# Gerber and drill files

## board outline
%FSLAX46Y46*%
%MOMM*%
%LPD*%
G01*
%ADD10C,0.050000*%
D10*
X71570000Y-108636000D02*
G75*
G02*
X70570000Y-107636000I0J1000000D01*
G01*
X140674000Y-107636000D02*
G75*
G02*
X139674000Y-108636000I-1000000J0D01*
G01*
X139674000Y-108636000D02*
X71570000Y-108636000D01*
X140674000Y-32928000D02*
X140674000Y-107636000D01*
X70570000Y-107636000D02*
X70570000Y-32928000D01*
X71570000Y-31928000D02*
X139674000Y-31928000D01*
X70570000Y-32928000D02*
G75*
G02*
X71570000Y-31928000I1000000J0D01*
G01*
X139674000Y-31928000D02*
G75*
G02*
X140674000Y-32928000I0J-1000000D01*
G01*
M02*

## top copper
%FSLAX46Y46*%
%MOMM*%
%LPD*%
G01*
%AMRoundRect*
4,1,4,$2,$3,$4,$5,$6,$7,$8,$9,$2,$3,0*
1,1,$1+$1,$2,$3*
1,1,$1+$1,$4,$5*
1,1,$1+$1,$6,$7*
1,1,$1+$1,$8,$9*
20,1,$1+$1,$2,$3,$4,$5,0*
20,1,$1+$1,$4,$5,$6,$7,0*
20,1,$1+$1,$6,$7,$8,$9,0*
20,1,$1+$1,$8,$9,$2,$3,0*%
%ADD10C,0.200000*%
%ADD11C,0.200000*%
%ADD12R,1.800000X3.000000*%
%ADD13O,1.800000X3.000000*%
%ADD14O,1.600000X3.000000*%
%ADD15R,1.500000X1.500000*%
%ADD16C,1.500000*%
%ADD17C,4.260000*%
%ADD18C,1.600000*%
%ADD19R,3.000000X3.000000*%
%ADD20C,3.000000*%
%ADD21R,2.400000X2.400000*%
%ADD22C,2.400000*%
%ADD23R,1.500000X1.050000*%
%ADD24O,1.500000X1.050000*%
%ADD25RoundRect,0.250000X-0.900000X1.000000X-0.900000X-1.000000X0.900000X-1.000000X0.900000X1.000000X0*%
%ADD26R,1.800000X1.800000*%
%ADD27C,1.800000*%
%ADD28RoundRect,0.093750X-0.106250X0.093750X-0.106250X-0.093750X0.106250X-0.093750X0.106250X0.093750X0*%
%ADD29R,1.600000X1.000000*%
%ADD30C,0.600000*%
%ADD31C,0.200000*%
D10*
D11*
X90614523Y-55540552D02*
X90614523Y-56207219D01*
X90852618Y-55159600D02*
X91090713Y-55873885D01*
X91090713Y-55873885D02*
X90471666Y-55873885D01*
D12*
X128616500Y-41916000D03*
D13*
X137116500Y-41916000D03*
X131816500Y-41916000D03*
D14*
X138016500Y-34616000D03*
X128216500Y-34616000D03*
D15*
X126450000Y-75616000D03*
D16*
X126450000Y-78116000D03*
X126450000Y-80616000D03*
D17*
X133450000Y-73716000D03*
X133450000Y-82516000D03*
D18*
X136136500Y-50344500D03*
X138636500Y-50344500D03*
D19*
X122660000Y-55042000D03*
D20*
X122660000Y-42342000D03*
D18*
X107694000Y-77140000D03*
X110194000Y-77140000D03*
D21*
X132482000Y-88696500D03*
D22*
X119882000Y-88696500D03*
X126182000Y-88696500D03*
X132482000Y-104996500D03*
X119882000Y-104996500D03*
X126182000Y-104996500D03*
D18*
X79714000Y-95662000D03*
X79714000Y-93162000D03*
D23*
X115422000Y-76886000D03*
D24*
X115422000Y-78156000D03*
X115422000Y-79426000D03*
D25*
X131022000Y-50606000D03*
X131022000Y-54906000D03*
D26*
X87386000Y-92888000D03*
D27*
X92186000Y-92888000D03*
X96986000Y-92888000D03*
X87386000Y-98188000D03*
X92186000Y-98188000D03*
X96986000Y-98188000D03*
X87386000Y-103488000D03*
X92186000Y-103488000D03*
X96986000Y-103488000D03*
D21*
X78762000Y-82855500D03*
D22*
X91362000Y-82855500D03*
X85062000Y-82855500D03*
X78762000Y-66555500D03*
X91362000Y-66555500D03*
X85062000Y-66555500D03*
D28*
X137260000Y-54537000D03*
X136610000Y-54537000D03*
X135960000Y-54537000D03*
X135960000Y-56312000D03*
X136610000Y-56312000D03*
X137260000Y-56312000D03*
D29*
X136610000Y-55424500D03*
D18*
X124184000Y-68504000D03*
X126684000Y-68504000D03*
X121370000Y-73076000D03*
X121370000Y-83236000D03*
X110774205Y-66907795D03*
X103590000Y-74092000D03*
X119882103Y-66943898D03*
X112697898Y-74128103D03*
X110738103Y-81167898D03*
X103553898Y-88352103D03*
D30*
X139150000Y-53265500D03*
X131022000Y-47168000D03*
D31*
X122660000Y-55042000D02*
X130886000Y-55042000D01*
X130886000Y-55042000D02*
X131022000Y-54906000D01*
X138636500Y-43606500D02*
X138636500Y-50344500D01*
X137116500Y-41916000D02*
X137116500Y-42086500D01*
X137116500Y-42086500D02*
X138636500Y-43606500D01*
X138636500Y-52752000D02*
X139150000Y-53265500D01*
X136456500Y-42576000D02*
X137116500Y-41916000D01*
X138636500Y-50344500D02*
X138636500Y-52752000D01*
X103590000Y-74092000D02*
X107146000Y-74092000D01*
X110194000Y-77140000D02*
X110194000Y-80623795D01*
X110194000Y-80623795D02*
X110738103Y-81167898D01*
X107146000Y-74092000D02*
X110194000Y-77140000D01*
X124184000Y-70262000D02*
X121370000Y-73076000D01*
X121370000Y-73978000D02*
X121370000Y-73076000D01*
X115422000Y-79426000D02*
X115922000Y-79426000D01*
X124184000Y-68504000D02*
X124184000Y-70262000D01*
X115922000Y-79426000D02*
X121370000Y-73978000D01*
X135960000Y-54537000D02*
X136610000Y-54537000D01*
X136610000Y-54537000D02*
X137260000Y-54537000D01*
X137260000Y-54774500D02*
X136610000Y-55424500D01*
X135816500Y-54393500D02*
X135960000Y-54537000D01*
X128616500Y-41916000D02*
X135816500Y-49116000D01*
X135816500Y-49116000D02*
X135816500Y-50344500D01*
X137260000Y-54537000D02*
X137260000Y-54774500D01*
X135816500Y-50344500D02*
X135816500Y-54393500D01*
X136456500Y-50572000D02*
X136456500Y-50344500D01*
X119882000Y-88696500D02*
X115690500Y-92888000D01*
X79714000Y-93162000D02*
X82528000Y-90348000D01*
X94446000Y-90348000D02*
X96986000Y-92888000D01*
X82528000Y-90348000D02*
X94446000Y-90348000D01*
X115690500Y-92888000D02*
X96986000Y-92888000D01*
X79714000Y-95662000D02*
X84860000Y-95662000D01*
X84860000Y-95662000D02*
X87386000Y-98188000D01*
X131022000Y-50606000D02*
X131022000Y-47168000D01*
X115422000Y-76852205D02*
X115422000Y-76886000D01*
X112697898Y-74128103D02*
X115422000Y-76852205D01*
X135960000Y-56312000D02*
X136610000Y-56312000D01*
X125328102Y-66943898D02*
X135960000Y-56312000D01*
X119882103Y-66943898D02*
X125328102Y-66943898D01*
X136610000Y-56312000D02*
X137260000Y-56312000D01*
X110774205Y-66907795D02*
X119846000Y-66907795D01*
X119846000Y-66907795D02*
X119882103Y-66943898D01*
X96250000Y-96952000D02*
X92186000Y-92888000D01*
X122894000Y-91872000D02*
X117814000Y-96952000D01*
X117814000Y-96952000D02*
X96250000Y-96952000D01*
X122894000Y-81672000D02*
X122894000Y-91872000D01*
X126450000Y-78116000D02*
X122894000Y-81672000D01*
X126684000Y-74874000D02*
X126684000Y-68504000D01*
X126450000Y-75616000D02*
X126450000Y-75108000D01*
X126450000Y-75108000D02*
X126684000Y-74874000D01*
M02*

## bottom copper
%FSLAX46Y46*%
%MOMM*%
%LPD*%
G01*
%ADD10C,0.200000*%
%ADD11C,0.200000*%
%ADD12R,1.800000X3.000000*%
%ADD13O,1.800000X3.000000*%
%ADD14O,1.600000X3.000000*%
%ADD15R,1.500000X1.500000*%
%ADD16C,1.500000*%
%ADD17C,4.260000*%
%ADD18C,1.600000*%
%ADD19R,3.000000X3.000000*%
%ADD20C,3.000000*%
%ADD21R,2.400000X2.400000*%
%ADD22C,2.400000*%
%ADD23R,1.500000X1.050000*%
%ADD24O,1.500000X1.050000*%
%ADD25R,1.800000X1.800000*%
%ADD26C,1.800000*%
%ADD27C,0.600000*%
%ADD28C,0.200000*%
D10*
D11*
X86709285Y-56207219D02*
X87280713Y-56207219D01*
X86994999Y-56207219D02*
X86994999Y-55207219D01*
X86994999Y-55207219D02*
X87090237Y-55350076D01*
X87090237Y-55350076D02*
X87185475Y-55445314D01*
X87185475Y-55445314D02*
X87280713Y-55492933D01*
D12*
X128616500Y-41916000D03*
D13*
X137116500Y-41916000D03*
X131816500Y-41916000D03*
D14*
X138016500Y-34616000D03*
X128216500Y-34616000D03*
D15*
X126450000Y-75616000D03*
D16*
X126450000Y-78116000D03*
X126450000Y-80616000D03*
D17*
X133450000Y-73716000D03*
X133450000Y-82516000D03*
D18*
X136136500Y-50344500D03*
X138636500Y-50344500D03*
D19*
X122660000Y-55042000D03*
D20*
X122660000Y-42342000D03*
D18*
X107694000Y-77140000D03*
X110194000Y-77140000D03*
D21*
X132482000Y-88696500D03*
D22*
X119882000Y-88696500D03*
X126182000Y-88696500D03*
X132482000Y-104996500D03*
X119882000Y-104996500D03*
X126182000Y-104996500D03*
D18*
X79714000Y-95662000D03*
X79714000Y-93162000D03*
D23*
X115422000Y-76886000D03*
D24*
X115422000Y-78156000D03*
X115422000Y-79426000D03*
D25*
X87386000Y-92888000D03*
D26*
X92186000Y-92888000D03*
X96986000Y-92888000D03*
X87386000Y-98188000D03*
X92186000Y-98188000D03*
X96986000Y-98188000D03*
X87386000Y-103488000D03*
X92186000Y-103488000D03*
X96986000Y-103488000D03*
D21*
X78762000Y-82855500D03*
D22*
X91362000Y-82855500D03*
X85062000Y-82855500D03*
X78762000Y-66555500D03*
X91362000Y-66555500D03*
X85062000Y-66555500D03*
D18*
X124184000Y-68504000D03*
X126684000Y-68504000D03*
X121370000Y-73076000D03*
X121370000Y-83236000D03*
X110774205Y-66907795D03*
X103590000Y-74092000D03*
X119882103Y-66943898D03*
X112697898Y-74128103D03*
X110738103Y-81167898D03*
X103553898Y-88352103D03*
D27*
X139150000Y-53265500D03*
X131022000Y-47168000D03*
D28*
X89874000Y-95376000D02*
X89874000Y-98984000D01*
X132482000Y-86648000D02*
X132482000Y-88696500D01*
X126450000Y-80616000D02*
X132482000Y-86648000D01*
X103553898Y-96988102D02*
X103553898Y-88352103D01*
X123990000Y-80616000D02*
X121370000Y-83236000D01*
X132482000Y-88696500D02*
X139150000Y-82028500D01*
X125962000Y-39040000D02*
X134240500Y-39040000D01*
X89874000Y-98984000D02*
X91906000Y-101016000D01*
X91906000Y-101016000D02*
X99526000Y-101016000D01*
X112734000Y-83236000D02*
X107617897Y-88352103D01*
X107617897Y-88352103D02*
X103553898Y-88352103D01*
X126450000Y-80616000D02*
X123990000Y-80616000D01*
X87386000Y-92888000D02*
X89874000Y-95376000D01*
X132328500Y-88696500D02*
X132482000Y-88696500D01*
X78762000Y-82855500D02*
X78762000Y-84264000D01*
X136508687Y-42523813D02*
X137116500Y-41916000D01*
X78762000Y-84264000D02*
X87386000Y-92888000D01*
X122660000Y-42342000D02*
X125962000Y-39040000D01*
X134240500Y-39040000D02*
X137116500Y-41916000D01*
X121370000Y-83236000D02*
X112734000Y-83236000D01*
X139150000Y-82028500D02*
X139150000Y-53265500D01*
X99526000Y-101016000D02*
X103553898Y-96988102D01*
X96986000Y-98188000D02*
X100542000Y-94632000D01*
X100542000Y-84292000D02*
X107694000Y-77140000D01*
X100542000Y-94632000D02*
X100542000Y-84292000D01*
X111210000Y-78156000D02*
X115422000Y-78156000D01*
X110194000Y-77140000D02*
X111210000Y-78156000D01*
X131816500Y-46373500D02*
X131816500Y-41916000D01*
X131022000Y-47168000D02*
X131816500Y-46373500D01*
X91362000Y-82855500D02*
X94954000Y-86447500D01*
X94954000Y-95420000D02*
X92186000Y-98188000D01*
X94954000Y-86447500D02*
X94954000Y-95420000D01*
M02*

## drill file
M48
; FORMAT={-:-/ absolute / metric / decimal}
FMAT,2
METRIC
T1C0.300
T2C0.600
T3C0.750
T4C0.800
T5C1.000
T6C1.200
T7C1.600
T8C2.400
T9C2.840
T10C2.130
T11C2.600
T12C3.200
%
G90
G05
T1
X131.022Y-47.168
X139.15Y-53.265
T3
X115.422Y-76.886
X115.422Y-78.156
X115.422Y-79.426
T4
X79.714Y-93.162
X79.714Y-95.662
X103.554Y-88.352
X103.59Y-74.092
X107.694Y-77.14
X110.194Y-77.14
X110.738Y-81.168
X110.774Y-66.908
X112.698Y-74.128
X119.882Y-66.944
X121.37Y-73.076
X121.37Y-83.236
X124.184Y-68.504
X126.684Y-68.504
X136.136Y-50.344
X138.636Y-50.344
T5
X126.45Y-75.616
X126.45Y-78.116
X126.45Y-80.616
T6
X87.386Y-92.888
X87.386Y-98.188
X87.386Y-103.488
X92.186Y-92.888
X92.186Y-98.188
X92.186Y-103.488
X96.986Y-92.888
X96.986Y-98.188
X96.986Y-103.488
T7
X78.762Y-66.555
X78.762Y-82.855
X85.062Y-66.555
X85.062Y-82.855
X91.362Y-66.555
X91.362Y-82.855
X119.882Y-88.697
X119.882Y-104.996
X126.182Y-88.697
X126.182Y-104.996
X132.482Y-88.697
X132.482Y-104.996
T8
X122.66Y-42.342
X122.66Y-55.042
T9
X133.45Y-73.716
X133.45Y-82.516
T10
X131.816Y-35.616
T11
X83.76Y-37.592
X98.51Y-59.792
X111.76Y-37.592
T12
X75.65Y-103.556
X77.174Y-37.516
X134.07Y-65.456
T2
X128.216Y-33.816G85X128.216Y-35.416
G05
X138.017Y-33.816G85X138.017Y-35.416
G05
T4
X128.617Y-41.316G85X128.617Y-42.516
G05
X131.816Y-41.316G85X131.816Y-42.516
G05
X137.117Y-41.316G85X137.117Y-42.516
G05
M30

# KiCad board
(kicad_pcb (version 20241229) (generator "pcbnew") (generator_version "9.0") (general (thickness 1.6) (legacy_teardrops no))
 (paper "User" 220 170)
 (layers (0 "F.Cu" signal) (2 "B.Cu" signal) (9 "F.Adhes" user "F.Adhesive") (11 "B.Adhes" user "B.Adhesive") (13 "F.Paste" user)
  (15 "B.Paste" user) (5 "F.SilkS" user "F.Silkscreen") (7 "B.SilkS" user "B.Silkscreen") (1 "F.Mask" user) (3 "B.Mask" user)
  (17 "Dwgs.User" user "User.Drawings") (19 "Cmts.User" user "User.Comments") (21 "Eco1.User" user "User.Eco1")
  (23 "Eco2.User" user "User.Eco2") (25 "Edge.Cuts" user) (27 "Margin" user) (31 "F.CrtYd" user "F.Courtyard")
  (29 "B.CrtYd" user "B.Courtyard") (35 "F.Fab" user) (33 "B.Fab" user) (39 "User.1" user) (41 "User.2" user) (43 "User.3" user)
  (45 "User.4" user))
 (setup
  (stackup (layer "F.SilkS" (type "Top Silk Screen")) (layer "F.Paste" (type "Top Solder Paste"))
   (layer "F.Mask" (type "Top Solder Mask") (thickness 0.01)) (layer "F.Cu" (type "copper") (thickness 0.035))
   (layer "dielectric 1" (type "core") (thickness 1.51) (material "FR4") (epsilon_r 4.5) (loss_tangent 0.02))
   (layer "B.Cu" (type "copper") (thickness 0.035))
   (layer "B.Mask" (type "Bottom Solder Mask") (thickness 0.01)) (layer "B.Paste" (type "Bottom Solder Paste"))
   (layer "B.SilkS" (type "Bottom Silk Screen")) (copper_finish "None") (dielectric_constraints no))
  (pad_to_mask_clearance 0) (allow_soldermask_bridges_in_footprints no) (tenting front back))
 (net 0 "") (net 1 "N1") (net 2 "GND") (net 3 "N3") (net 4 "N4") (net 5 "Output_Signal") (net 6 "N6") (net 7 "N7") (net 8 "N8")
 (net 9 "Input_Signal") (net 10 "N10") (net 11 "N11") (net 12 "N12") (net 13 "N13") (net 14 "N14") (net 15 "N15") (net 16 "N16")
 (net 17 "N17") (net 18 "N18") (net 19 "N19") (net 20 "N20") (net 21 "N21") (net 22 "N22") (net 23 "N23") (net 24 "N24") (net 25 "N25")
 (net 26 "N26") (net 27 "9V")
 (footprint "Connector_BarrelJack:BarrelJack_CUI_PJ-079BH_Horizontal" (layer "F.Cu") (at 128.6165 41.916 180)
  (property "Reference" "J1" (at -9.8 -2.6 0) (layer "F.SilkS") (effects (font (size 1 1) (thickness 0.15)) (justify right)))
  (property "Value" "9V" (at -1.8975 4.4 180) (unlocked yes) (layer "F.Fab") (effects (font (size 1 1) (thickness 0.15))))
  (pad "" np_thru_hole circle (at -3.2 6.3) (size 2.13 2.13) (drill 2.13) (layers "*.Cu" "*.Mask"))
  (pad "1" thru_hole rect (at 0 0) (size 1.8 3) (drill oval 0.8 2) (layers "*.Cu" "*.Mask") (remove_unused_layers no) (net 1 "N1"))
  (pad "2" thru_hole oval (at -8.5 0) (size 1.8 3) (drill oval 0.8 2) (layers "*.Cu" "*.Mask") (remove_unused_layers no) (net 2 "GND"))
  (pad "3" thru_hole oval (at -3.2 0) (size 1.8 3) (drill oval 0.8 2) (layers "*.Cu" "*.Mask") (remove_unused_layers no) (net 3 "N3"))
  (pad "SH" thru_hole oval (at -9.4 7.3) (size 1.6 3) (drill oval 0.6 2.2) (layers "*.Cu" "*.Mask") (remove_unused_layers no))
  (pad "SH" thru_hole oval (at 0.4 7.3) (size 1.6 3) (drill oval 0.6 2.2) (layers "*.Cu" "*.Mask") (remove_unused_layers no)))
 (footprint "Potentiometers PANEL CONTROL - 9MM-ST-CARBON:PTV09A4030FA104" (layer "F.Cu") (at 126.45 75.616 -90)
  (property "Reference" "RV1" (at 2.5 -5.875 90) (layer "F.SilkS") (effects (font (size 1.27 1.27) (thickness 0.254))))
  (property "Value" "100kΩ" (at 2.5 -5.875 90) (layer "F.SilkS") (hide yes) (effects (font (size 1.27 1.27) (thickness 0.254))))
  (pad "1" thru_hole rect (at 0 0 270) (size 1.5 1.5) (drill 1) (layers "*.Cu" "*.Mask") (remove_unused_layers no) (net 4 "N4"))
  (pad "2" thru_hole circle (at 2.5 0 270) (size 1.5 1.5) (drill 1) (layers "*.Cu" "*.Mask") (remove_unused_layers no)
   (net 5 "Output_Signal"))
  (pad "3" thru_hole circle (at 5 0 270) (size 1.5 1.5) (drill 1) (layers "*.Cu" "*.Mask") (remove_unused_layers no) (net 2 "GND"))
  (pad "4" thru_hole circle (at -1.9 -7 270) (size 4.26 4.26) (drill 2.84) (layers "*.Cu" "*.Mask") (remove_unused_layers no) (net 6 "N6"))
  (pad "5" thru_hole circle (at 6.9 -7 270) (size 4.26 4.26) (drill 2.84) (layers "*.Cu" "*.Mask") (remove_unused_layers no) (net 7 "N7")))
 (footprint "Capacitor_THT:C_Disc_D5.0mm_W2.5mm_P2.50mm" (layer "F.Cu") (at 136.1365 50.3445)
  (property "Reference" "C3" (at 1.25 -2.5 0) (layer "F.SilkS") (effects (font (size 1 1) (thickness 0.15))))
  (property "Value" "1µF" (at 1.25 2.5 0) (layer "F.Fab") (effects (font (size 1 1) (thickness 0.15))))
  (pad "1" thru_hole circle (at 0 0) (size 1.6 1.6) (drill 0.8) (layers "*.Cu" "*.Mask") (remove_unused_layers no) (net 1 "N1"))
  (pad "2" thru_hole circle (at 2.5 0) (size 1.6 1.6) (drill 0.8) (layers "*.Cu" "*.Mask") (remove_unused_layers no) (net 2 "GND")))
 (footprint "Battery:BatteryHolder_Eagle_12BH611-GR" (layer "F.Cu") (at 122.66 55.042)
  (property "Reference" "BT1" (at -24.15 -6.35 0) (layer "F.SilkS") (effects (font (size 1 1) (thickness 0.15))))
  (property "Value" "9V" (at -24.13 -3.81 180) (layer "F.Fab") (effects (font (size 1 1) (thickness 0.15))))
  (pad "" np_thru_hole circle (at -38.9 -17.45) (size 2.6 2.6) (drill 2.6) (layers "*.Cu" "*.Mask"))
  (pad "" np_thru_hole circle (at -24.15 4.75) (size 2.6 2.6) (drill 2.6) (layers "*.Cu" "*.Mask"))
  (pad "" np_thru_hole circle (at -10.9 -17.45) (size 2.6 2.6) (drill 2.6) (layers "*.Cu" "*.Mask"))
  (pad "1" thru_hole rect (at 0 0) (size 3 3) (drill 2.4) (layers "*.Cu" "*.Mask") (remove_unused_layers no) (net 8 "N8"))
  (pad "2" thru_hole circle (at 0 -12.7) (size 3 3) (drill 2.4) (layers "*.Cu" "*.Mask") (remove_unused_layers no) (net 2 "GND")))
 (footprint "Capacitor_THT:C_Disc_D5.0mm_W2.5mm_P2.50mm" (layer "F.Cu") (at 107.694 77.14)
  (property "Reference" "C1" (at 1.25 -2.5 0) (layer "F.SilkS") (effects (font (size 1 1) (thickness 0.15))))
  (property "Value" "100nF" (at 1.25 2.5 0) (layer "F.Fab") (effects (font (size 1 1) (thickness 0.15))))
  (pad "1" thru_hole circle (at 0 0) (size 1.6 1.6) (drill 0.8) (layers "*.Cu" "*.Mask") (remove_unused_layers no) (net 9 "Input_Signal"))
  (pad "2" thru_hole circle (at 2.5 0) (size 1.6 1.6) (drill 0.8) (layers "*.Cu" "*.Mask") (remove_unused_layers no) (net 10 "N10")))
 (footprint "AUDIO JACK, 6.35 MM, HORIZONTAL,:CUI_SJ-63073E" (layer "F.Cu") (at 132.482 96.8465 180)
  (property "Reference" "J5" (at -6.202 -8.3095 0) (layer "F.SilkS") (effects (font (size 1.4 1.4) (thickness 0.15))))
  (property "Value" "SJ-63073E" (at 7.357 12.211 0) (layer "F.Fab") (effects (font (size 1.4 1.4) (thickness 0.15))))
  (pad "1" thru_hole rect (at 0 8.15 180) (size 2.4 2.4) (drill 1.6) (layers "*.Cu" "*.Mask") (remove_unused_layers no) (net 2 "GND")
   (solder_mask_margin 0.102))
  (pad "2" thru_hole circle (at 12.6 8.15 180) (size 2.4 2.4) (drill 1.6) (layers "*.Cu" "*.Mask") (remove_unused_layers no) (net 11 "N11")
   (solder_mask_margin 0.102))
  (pad "3" thru_hole circle (at 6.3 8.15 180) (size 2.4 2.4) (drill 1.6) (layers "*.Cu" "*.Mask") (remove_unused_layers no) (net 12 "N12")
   (solder_mask_margin 0.102))
  (pad "4" thru_hole circle (at 0 -8.15 180) (size 2.4 2.4) (drill 1.6) (layers "*.Cu" "*.Mask") (remove_unused_layers no) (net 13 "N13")
   (solder_mask_margin 0.102))
  (pad "5" thru_hole circle (at 12.6 -8.15 180) (size 2.4 2.4) (drill 1.6) (layers "*.Cu" "*.Mask") (remove_unused_layers no) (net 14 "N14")
   (solder_mask_margin 0.102))
  (pad "6" thru_hole circle (at 6.3 -8.15 180) (size 2.4 2.4) (drill 1.6) (layers "*.Cu" "*.Mask") (remove_unused_layers no) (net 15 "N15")
   (solder_mask_margin 0.102)))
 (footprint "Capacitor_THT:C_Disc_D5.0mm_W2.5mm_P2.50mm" (layer "F.Cu") (at 79.714 95.662 90)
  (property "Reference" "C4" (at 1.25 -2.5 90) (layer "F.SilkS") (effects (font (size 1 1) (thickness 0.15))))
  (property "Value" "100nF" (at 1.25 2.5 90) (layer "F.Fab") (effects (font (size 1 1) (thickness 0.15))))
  (pad "1" thru_hole circle (at 0 0 90) (size 1.6 1.6) (drill 0.8) (layers "*.Cu" "*.Mask") (remove_unused_layers no) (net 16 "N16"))
  (pad "2" thru_hole circle (at 2.5 0 90) (size 1.6 1.6) (drill 0.8) (layers "*.Cu" "*.Mask") (remove_unused_layers no) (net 11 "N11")))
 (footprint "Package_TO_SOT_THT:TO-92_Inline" (layer "F.Cu") (at 115.422 76.886 -90)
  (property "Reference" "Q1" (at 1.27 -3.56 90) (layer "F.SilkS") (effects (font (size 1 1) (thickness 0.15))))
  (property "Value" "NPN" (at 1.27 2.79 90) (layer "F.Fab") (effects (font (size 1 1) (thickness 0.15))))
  (pad "1" thru_hole rect (at 0 0 270) (size 1.05 1.5) (drill 0.75) (layers "*.Cu" "*.Mask") (remove_unused_layers no) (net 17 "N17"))
  (pad "2" thru_hole oval (at 1.27 0 270) (size 1.05 1.5) (drill 0.75) (layers "*.Cu" "*.Mask") (remove_unused_layers no) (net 10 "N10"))
  (pad "3" thru_hole oval (at 2.54 0 270) (size 1.05 1.5) (drill 0.75) (layers "*.Cu" "*.Mask") (remove_unused_layers no) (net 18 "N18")))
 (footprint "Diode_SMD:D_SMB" (layer "F.Cu") (at 131.022 52.756 -90)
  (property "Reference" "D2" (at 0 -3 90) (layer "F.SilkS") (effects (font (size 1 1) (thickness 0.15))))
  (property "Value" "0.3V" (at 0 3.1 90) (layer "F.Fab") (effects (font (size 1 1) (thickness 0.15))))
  (pad "1" smd roundrect (at -2.15 0 270) (size 2.5 2.3) (layers "F.Cu" "F.Mask" "F.Paste") (roundrect_rratio 0.1086956522) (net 3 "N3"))
  (pad "2" smd roundrect (at 2.15 0 270) (size 2.5 2.3) (layers "F.Cu" "F.Mask" "F.Paste") (roundrect_rratio 0.1086956522) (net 8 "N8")))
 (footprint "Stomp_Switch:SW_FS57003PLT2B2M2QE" (layer "F.Cu") (at 92.186 98.188 -90)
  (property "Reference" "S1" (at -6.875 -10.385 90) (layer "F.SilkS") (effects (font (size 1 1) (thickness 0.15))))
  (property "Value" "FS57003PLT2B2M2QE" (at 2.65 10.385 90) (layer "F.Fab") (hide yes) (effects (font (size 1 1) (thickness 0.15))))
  (pad "1" thru_hole rect (at -5.3 4.8 270) (size 1.8 1.8) (drill 1.2) (layers "*.Cu" "*.Mask") (remove_unused_layers no) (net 2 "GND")
   (solder_mask_margin 0.102))
  (pad "2" thru_hole circle (at -5.3 0 270) (size 1.8 1.8) (drill 1.2) (layers "*.Cu" "*.Mask") (remove_unused_layers no)
   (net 5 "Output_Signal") (solder_mask_margin 0.102))
  (pad "3" thru_hole circle (at -5.3 -4.8 270) (size 1.8 1.8) (drill 1.2) (layers "*.Cu" "*.Mask") (remove_unused_layers no) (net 11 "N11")
   (solder_mask_margin 0.102))
  (pad "4" thru_hole circle (at 0 4.8 270) (size 1.8 1.8) (drill 1.2) (layers "*.Cu" "*.Mask") (remove_unused_layers no) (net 16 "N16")
   (solder_mask_margin 0.102))
  (pad "5" thru_hole circle (at 0 0 270) (size 1.8 1.8) (drill 1.2) (layers "*.Cu" "*.Mask") (remove_unused_layers no) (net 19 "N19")
   (solder_mask_margin 0.102))
  (pad "6" thru_hole circle (at 0 -4.8 270) (size 1.8 1.8) (drill 1.2) (layers "*.Cu" "*.Mask") (remove_unused_layers no)
   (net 9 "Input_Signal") (solder_mask_margin 0.102))
  (pad "7" thru_hole circle (at 5.3 4.8 270) (size 1.8 1.8) (drill 1.2) (layers "*.Cu" "*.Mask") (remove_unused_layers no) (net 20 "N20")
   (solder_mask_margin 0.102))
  (pad "8" thru_hole circle (at 5.3 0 270) (size 1.8 1.8) (drill 1.2) (layers "*.Cu" "*.Mask") (remove_unused_layers no) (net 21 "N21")
   (solder_mask_margin 0.102))
  (pad "9" thru_hole circle (at 5.3 -4.8 270) (size 1.8 1.8) (drill 1.2) (layers "*.Cu" "*.Mask") (remove_unused_layers no) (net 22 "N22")
   (solder_mask_margin 0.102)))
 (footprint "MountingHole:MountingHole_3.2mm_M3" (layer "F.Cu") (at 75.65 103.556)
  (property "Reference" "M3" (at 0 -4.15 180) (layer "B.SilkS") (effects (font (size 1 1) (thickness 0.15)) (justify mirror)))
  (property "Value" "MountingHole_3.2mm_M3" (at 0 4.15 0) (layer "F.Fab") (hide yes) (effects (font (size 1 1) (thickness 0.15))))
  (pad "" np_thru_hole circle (at 0 0) (size 3.2 3.2) (drill 3.2) (layers "*.Cu" "*.Mask")))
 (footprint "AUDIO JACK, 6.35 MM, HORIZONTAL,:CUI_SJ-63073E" (layer "F.Cu") (at 78.762 74.7055)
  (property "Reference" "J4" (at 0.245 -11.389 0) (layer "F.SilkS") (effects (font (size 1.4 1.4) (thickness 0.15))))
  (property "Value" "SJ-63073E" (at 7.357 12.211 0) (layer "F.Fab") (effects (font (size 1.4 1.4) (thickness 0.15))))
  (pad "1" thru_hole rect (at 0 8.15) (size 2.4 2.4) (drill 1.6) (layers "*.Cu" "*.Mask") (remove_unused_layers no) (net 2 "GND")
   (solder_mask_margin 0.102))
  (pad "2" thru_hole circle (at 12.6 8.15) (size 2.4 2.4) (drill 1.6) (layers "*.Cu" "*.Mask") (remove_unused_layers no) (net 19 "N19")
   (solder_mask_margin 0.102))
  (pad "3" thru_hole circle (at 6.3 8.15) (size 2.4 2.4) (drill 1.6) (layers "*.Cu" "*.Mask") (remove_unused_layers no) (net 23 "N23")
   (solder_mask_margin 0.102))
  (pad "4" thru_hole circle (at 0 -8.15) (size 2.4 2.4) (drill 1.6) (layers "*.Cu" "*.Mask") (remove_unused_layers no) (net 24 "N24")
   (solder_mask_margin 0.102))
  (pad "5" thru_hole circle (at 12.6 -8.15) (size 2.4 2.4) (drill 1.6) (layers "*.Cu" "*.Mask") (remove_unused_layers no) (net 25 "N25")
   (solder_mask_margin 0.102))
  (pad "6" thru_hole circle (at 6.3 -8.15) (size 2.4 2.4) (drill 1.6) (layers "*.Cu" "*.Mask") (remove_unused_layers no) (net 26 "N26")
   (solder_mask_margin 0.102)))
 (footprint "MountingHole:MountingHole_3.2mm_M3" (layer "F.Cu") (at 134.07 65.456)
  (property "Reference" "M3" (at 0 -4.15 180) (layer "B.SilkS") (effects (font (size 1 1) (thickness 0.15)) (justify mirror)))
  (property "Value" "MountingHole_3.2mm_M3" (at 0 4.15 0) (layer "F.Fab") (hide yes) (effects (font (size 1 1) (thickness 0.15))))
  (pad "" np_thru_hole circle (at 0 0) (size 3.2 3.2) (drill 3.2) (layers "*.Cu" "*.Mask")))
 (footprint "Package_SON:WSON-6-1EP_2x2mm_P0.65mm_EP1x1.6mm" (layer "F.Cu") (at 136.61 55.4245 -90)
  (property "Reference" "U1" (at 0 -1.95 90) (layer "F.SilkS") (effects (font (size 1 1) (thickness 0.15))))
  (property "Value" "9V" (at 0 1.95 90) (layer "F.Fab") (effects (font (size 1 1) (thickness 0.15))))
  (pad "" smd roundrect (at 0 -0.4 270) (size 0.81 0.64) (layers "F.Paste") (roundrect_rratio 0.25))
  (pad "" smd roundrect (at 0 0.4 270) (size 0.81 0.64) (layers "F.Paste") (roundrect_rratio 0.25))
  (pad "1" smd roundrect (at -0.8875 -0.65 270) (size 0.375 0.4) (layers "F.Cu" "F.Mask" "F.Paste") (roundrect_rratio 0.25) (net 1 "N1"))
  (pad "2" smd roundrect (at -0.8875 0 270) (size 0.375 0.4) (layers "F.Cu" "F.Mask" "F.Paste") (roundrect_rratio 0.25) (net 1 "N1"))
  (pad "3" smd roundrect (at -0.8875 0.65 270) (size 0.375 0.4) (layers "F.Cu" "F.Mask" "F.Paste") (roundrect_rratio 0.25) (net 1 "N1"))
  (pad "4" smd roundrect (at 0.8875 0.65 270) (size 0.375 0.4) (layers "F.Cu" "F.Mask" "F.Paste") (roundrect_rratio 0.25) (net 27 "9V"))
  (pad "5" smd roundrect (at 0.8875 0 270) (size 0.375 0.4) (layers "F.Cu" "F.Mask" "F.Paste") (roundrect_rratio 0.25) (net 27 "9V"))
  (pad "6" smd roundrect (at 0.8875 -0.65 270) (size 0.375 0.4) (layers "F.Cu" "F.Mask" "F.Paste") (roundrect_rratio 0.25) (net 27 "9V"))
  (pad "7" smd rect (at 0 0 270) (size 1 1.6) (layers "F.Cu" "F.Mask") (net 1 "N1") (zone_connect 2)))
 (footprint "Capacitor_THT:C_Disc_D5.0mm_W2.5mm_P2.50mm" (layer "F.Cu") (at 124.184 68.504)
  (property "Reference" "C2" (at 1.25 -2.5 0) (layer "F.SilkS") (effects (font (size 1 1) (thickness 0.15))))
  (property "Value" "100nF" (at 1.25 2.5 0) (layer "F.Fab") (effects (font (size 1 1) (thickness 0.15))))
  (pad "1" thru_hole circle (at 0 0) (size 1.6 1.6) (drill 0.8) (layers "*.Cu" "*.Mask") (remove_unused_layers no) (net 18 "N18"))
  (pad "2" thru_hole circle (at 2.5 0) (size 1.6 1.6) (drill 0.8) (layers "*.Cu" "*.Mask") (remove_unused_layers no) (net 4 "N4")))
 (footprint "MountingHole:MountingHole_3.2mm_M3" (layer "B.Cu") (at 77.174 37.516)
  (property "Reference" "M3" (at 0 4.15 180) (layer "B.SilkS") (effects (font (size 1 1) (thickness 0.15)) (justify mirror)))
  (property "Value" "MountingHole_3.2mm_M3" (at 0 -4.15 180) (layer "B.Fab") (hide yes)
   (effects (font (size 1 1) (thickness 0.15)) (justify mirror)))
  (pad "" np_thru_hole circle (at 0 0) (size 3.2 3.2) (drill 3.2) (layers "*.Cu" "*.Mask")))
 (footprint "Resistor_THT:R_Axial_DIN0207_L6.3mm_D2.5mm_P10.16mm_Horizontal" (layer "B.Cu") (at 121.37 73.076 -90)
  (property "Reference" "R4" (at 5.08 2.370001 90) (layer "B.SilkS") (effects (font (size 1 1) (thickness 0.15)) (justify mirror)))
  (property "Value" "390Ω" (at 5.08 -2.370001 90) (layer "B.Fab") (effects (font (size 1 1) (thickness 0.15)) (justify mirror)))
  (pad "1" thru_hole circle (at 0 0 270) (size 1.6 1.6) (drill 0.8) (layers "*.Cu" "*.Mask") (remove_unused_layers no) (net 18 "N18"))
  (pad "2" thru_hole circle (at 10.16 0 270) (size 1.6 1.6) (drill 0.8) (layers "*.Cu" "*.Mask") (remove_unused_layers no) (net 2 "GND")))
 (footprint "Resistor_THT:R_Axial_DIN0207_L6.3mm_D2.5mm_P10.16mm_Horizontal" (layer "B.Cu") (at 110.774205 66.907795 -135)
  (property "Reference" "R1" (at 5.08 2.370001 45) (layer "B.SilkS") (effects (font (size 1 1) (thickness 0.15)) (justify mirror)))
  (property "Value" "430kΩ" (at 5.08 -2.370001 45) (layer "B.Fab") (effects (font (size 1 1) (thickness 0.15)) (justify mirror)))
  (pad "1" thru_hole circle (at 0 0 225) (size 1.6 1.6) (drill 0.8) (layers "*.Cu" "*.Mask") (remove_unused_layers no) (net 27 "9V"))
  (pad "2" thru_hole circle (at 10.16 0 225) (size 1.6 1.6) (drill 0.8) (layers "*.Cu" "*.Mask") (remove_unused_layers no) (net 10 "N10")))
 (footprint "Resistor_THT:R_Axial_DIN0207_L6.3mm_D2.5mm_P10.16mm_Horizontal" (layer "B.Cu") (at 119.882103 66.943898 -135)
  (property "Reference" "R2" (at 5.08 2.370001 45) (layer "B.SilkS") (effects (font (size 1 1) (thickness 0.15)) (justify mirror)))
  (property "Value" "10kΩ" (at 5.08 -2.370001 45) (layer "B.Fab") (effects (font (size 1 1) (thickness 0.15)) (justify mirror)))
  (pad "1" thru_hole circle (at 0 0 225) (size 1.6 1.6) (drill 0.8) (layers "*.Cu" "*.Mask") (remove_unused_layers no) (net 27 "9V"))
  (pad "2" thru_hole circle (at 10.16 0 225) (size 1.6 1.6) (drill 0.8) (layers "*.Cu" "*.Mask") (remove_unused_layers no) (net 17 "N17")))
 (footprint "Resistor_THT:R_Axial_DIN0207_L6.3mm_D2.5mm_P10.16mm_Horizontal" (layer "B.Cu") (at 110.738103 81.167898 -135)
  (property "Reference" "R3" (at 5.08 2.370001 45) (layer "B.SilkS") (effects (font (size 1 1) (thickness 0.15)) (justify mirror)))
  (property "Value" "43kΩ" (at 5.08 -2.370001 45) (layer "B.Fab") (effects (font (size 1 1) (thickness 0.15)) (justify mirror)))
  (pad "1" thru_hole circle (at 0 0 225) (size 1.6 1.6) (drill 0.8) (layers "*.Cu" "*.Mask") (remove_unused_layers no) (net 10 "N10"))
  (pad "2" thru_hole circle (at 10.16 0 225) (size 1.6 1.6) (drill 0.8) (layers "*.Cu" "*.Mask") (remove_unused_layers no) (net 2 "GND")))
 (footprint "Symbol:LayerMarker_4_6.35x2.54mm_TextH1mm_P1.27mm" (layer "B.Cu") (at 86.995 54.485)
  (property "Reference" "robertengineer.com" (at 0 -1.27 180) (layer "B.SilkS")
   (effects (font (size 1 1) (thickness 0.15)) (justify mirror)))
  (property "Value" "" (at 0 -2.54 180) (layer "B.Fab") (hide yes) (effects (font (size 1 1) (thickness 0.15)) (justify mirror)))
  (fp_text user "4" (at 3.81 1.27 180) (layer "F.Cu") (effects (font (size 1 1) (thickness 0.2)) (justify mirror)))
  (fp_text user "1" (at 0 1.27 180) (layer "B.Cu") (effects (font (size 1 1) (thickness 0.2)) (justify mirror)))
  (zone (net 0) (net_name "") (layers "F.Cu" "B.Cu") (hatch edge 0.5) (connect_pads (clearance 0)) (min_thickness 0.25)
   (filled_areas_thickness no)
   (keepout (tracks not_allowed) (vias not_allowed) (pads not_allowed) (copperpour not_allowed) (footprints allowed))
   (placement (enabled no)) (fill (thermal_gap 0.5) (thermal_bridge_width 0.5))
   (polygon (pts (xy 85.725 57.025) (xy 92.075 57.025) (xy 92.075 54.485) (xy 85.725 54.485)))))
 (gr_arc (start 71.57 108.636) (mid 70.862893 108.343107) (end 70.57 107.636) (stroke (width 0.05) (type default)) (layer "Edge.Cuts"))
 (gr_arc (start 140.674 107.636) (mid 140.381107 108.343107) (end 139.674 108.636) (stroke (width 0.05) (type default)) (layer "Edge.Cuts"))
 (gr_line (start 139.674 108.636) (end 71.57 108.636) (stroke (width 0.05) (type default)) (layer "Edge.Cuts"))
 (gr_line (start 140.674 32.928) (end 140.674 107.636) (stroke (width 0.05) (type default)) (layer "Edge.Cuts"))
 (gr_line (start 70.57 107.636) (end 70.57 32.928) (stroke (width 0.05) (type default)) (layer "Edge.Cuts"))
 (gr_line (start 71.57 31.928) (end 139.674 31.928) (stroke (width 0.05) (type default)) (layer "Edge.Cuts"))
 (gr_arc (start 70.57 32.928) (mid 70.862893 32.220893) (end 71.57 31.928) (stroke (width 0.05) (type default)) (layer "Edge.Cuts"))
 (gr_arc (start 139.674 31.928) (mid 140.381107 32.220893) (end 140.674 32.928) (stroke (width 0.05) (type default)) (layer "Edge.Cuts"))
 (segment (start 122.66 55.042) (end 130.886 55.042) (width 0.2) (layer "F.Cu") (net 8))
 (segment (start 130.886 55.042) (end 131.022 54.906) (width 0.2) (layer "F.Cu") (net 8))
 (segment (start 138.6365 43.6065) (end 138.6365 50.3445) (width 0.2) (layer "F.Cu") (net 2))
 (segment (start 137.1165 41.916) (end 137.1165 42.0865) (width 0.2) (layer "F.Cu") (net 2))
 (segment (start 137.1165 42.0865) (end 138.6365 43.6065) (width 0.2) (layer "F.Cu") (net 2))
 (segment (start 138.6365 52.752) (end 139.15 53.2655) (width 0.2) (layer "F.Cu") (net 2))
 (segment (start 136.4565 42.576) (end 137.1165 41.916) (width 0.2) (layer "F.Cu") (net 2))
 (segment (start 138.6365 50.3445) (end 138.6365 52.752) (width 0.2) (layer "F.Cu") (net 2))
 (via (at 139.15 53.2655) (size 0.6) (drill 0.3) (layers "F.Cu" "B.Cu") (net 2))
 (segment (start 89.874 95.376) (end 89.874 98.984) (width 0.2) (layer "B.Cu") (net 2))
 (segment (start 132.482 86.648) (end 132.482 88.6965) (width 0.2) (layer "B.Cu") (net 2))
 (segment (start 126.45 80.616) (end 132.482 86.648) (width 0.2) (layer "B.Cu") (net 2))
 (segment (start 103.553898 96.988102) (end 103.553898 88.352103) (width 0.2) (layer "B.Cu") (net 2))
 (segment (start 123.99 80.616) (end 121.37 83.236) (width 0.2) (layer "B.Cu") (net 2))
 (segment (start 132.482 88.6965) (end 139.15 82.0285) (width 0.2) (layer "B.Cu") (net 2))
 (segment (start 125.962 39.04) (end 134.2405 39.04) (width 0.2) (layer "B.Cu") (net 2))
 (segment (start 89.874 98.984) (end 91.906 101.016) (width 0.2) (layer "B.Cu") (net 2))
 (segment (start 91.906 101.016) (end 99.526 101.016) (width 0.2) (layer "B.Cu") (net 2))
 (segment (start 112.734 83.236) (end 107.617897 88.352103) (width 0.2) (layer "B.Cu") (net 2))
 (segment (start 107.617897 88.352103) (end 103.553898 88.352103) (width 0.2) (layer "B.Cu") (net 2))
 (segment (start 126.45 80.616) (end 123.99 80.616) (width 0.2) (layer "B.Cu") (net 2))
 (segment (start 87.386 92.888) (end 89.874 95.376) (width 0.2) (layer "B.Cu") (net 2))
 (segment (start 132.3285 88.6965) (end 132.482 88.6965) (width 0.2) (layer "B.Cu") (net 2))
 (segment (start 78.762 82.8555) (end 78.762 84.264) (width 0.2) (layer "B.Cu") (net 2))
 (segment (start 136.508687 42.523813) (end 137.1165 41.916) (width 0.2) (layer "B.Cu") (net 2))
 (segment (start 78.762 84.264) (end 87.386 92.888) (width 0.2) (layer "B.Cu") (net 2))
 (segment (start 122.66 42.342) (end 125.962 39.04) (width 0.2) (layer "B.Cu") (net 2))
 (segment (start 134.2405 39.04) (end 137.1165 41.916) (width 0.2) (layer "B.Cu") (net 2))
 (segment (start 121.37 83.236) (end 112.734 83.236) (width 0.2) (layer "B.Cu") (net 2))
 (segment (start 139.15 82.0285) (end 139.15 53.2655) (width 0.2) (layer "B.Cu") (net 2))
 (segment (start 99.526 101.016) (end 103.553898 96.988102) (width 0.2) (layer "B.Cu") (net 2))
 (segment (start 96.986 98.188) (end 100.542 94.632) (width 0.2) (layer "B.Cu") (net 9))
 (segment (start 100.542 84.292) (end 107.694 77.14) (width 0.2) (layer "B.Cu") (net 9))
 (segment (start 100.542 94.632) (end 100.542 84.292) (width 0.2) (layer "B.Cu") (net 9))
 (segment (start 103.59 74.092) (end 107.146 74.092) (width 0.2) (layer "F.Cu") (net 10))
 (segment (start 110.194 77.14) (end 110.194 80.623795) (width 0.2) (layer "F.Cu") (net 10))
 (segment (start 110.194 80.623795) (end 110.738103 81.167898) (width 0.2) (layer "F.Cu") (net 10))
 (segment (start 107.146 74.092) (end 110.194 77.14) (width 0.2) (layer "F.Cu") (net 10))
 (segment (start 111.21 78.156) (end 115.422 78.156) (width 0.2) (layer "B.Cu") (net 10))
 (segment (start 110.194 77.14) (end 111.21 78.156) (width 0.2) (layer "B.Cu") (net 10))
 (segment (start 124.184 70.262) (end 121.37 73.076) (width 0.2) (layer "F.Cu") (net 18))
 (segment (start 121.37 73.978) (end 121.37 73.076) (width 0.2) (layer "F.Cu") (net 18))
 (segment (start 115.422 79.426) (end 115.922 79.426) (width 0.2) (layer "F.Cu") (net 18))
 (segment (start 124.184 68.504) (end 124.184 70.262) (width 0.2) (layer "F.Cu") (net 18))
 (segment (start 115.922 79.426) (end 121.37 73.978) (width 0.2) (layer "F.Cu") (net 18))
 (segment (start 135.96 54.537) (end 136.61 54.537) (width 0.2) (layer "F.Cu") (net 1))
 (segment (start 136.61 54.537) (end 137.26 54.537) (width 0.2) (layer "F.Cu") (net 1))
 (segment (start 137.26 54.7745) (end 136.61 55.4245) (width 0.2) (layer "F.Cu") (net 1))
 (segment (start 135.8165 54.3935) (end 135.96 54.537) (width 0.2) (layer "F.Cu") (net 1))
 (segment (start 128.6165 41.916) (end 135.8165 49.116) (width 0.2) (layer "F.Cu") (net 1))
 (segment (start 135.8165 49.116) (end 135.8165 50.3445) (width 0.2) (layer "F.Cu") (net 1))
 (segment (start 137.26 54.537) (end 137.26 54.7745) (width 0.2) (layer "F.Cu") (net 1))
 (segment (start 135.8165 50.3445) (end 135.8165 54.3935) (width 0.2) (layer "F.Cu") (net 1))
 (segment (start 136.4565 50.572) (end 136.4565 50.3445) (width 0.2) (layer "F.Cu") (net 1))
 (segment (start 119.882 88.6965) (end 115.6905 92.888) (width 0.2) (layer "F.Cu") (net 11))
 (segment (start 79.714 93.162) (end 82.528 90.348) (width 0.2) (layer "F.Cu") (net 11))
 (segment (start 94.446 90.348) (end 96.986 92.888) (width 0.2) (layer "F.Cu") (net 11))
 (segment (start 82.528 90.348) (end 94.446 90.348) (width 0.2) (layer "F.Cu") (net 11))
 (segment (start 115.6905 92.888) (end 96.986 92.888) (width 0.2) (layer "F.Cu") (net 11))
 (segment (start 79.714 95.662) (end 84.86 95.662) (width 0.2) (layer "F.Cu") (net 16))
 (segment (start 84.86 95.662) (end 87.386 98.188) (width 0.2) (layer "F.Cu") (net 16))
 (segment (start 131.022 50.606) (end 131.022 47.168) (width 0.2) (layer "F.Cu") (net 3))
 (via (at 131.022 47.168) (size 0.6) (drill 0.3) (layers "F.Cu" "B.Cu") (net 3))
 (segment (start 131.8165 46.3735) (end 131.8165 41.916) (width 0.2) (layer "B.Cu") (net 3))
 (segment (start 131.022 47.168) (end 131.8165 46.3735) (width 0.2) (layer "B.Cu") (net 3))
 (segment (start 115.422 76.852205) (end 115.422 76.886) (width 0.2) (layer "F.Cu") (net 17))
 (segment (start 112.697898 74.128103) (end 115.422 76.852205) (width 0.2) (layer "F.Cu") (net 17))
 (segment (start 135.96 56.312) (end 136.61 56.312) (width 0.2) (layer "F.Cu") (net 27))
 (segment (start 125.328102 66.943898) (end 135.96 56.312) (width 0.2) (layer "F.Cu") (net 27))
 (segment (start 119.882103 66.943898) (end 125.328102 66.943898) (width 0.2) (layer "F.Cu") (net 27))
 (segment (start 136.61 56.312) (end 137.26 56.312) (width 0.2) (layer "F.Cu") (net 27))
 (segment (start 110.774205 66.907795) (end 119.846 66.907795) (width 0.2) (layer "F.Cu") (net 27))
 (segment (start 119.846 66.907795) (end 119.882103 66.943898) (width 0.2) (layer "F.Cu") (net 27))
 (segment (start 96.25 96.952) (end 92.186 92.888) (width 0.2) (layer "F.Cu") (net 5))
 (segment (start 122.894 91.872) (end 117.814 96.952) (width 0.2) (layer "F.Cu") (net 5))
 (segment (start 117.814 96.952) (end 96.25 96.952) (width 0.2) (layer "F.Cu") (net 5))
 (segment (start 122.894 81.672) (end 122.894 91.872) (width 0.2) (layer "F.Cu") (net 5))
 (segment (start 126.45 78.116) (end 122.894 81.672) (width 0.2) (layer "F.Cu") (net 5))
 (segment (start 91.362 82.8555) (end 94.954 86.4475) (width 0.2) (layer "B.Cu") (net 19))
 (segment (start 94.954 95.42) (end 92.186 98.188) (width 0.2) (layer "B.Cu") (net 19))
 (segment (start 94.954 86.4475) (end 94.954 95.42) (width 0.2) (layer "B.Cu") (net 19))
 (segment (start 126.684 74.874) (end 126.684 68.504) (width 0.2) (layer "F.Cu") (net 4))
 (segment (start 126.45 75.616) (end 126.45 75.108) (width 0.2) (layer "F.Cu") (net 4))
 (segment (start 126.45 75.108) (end 126.684 74.874) (width 0.2) (layer "F.Cu") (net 4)))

